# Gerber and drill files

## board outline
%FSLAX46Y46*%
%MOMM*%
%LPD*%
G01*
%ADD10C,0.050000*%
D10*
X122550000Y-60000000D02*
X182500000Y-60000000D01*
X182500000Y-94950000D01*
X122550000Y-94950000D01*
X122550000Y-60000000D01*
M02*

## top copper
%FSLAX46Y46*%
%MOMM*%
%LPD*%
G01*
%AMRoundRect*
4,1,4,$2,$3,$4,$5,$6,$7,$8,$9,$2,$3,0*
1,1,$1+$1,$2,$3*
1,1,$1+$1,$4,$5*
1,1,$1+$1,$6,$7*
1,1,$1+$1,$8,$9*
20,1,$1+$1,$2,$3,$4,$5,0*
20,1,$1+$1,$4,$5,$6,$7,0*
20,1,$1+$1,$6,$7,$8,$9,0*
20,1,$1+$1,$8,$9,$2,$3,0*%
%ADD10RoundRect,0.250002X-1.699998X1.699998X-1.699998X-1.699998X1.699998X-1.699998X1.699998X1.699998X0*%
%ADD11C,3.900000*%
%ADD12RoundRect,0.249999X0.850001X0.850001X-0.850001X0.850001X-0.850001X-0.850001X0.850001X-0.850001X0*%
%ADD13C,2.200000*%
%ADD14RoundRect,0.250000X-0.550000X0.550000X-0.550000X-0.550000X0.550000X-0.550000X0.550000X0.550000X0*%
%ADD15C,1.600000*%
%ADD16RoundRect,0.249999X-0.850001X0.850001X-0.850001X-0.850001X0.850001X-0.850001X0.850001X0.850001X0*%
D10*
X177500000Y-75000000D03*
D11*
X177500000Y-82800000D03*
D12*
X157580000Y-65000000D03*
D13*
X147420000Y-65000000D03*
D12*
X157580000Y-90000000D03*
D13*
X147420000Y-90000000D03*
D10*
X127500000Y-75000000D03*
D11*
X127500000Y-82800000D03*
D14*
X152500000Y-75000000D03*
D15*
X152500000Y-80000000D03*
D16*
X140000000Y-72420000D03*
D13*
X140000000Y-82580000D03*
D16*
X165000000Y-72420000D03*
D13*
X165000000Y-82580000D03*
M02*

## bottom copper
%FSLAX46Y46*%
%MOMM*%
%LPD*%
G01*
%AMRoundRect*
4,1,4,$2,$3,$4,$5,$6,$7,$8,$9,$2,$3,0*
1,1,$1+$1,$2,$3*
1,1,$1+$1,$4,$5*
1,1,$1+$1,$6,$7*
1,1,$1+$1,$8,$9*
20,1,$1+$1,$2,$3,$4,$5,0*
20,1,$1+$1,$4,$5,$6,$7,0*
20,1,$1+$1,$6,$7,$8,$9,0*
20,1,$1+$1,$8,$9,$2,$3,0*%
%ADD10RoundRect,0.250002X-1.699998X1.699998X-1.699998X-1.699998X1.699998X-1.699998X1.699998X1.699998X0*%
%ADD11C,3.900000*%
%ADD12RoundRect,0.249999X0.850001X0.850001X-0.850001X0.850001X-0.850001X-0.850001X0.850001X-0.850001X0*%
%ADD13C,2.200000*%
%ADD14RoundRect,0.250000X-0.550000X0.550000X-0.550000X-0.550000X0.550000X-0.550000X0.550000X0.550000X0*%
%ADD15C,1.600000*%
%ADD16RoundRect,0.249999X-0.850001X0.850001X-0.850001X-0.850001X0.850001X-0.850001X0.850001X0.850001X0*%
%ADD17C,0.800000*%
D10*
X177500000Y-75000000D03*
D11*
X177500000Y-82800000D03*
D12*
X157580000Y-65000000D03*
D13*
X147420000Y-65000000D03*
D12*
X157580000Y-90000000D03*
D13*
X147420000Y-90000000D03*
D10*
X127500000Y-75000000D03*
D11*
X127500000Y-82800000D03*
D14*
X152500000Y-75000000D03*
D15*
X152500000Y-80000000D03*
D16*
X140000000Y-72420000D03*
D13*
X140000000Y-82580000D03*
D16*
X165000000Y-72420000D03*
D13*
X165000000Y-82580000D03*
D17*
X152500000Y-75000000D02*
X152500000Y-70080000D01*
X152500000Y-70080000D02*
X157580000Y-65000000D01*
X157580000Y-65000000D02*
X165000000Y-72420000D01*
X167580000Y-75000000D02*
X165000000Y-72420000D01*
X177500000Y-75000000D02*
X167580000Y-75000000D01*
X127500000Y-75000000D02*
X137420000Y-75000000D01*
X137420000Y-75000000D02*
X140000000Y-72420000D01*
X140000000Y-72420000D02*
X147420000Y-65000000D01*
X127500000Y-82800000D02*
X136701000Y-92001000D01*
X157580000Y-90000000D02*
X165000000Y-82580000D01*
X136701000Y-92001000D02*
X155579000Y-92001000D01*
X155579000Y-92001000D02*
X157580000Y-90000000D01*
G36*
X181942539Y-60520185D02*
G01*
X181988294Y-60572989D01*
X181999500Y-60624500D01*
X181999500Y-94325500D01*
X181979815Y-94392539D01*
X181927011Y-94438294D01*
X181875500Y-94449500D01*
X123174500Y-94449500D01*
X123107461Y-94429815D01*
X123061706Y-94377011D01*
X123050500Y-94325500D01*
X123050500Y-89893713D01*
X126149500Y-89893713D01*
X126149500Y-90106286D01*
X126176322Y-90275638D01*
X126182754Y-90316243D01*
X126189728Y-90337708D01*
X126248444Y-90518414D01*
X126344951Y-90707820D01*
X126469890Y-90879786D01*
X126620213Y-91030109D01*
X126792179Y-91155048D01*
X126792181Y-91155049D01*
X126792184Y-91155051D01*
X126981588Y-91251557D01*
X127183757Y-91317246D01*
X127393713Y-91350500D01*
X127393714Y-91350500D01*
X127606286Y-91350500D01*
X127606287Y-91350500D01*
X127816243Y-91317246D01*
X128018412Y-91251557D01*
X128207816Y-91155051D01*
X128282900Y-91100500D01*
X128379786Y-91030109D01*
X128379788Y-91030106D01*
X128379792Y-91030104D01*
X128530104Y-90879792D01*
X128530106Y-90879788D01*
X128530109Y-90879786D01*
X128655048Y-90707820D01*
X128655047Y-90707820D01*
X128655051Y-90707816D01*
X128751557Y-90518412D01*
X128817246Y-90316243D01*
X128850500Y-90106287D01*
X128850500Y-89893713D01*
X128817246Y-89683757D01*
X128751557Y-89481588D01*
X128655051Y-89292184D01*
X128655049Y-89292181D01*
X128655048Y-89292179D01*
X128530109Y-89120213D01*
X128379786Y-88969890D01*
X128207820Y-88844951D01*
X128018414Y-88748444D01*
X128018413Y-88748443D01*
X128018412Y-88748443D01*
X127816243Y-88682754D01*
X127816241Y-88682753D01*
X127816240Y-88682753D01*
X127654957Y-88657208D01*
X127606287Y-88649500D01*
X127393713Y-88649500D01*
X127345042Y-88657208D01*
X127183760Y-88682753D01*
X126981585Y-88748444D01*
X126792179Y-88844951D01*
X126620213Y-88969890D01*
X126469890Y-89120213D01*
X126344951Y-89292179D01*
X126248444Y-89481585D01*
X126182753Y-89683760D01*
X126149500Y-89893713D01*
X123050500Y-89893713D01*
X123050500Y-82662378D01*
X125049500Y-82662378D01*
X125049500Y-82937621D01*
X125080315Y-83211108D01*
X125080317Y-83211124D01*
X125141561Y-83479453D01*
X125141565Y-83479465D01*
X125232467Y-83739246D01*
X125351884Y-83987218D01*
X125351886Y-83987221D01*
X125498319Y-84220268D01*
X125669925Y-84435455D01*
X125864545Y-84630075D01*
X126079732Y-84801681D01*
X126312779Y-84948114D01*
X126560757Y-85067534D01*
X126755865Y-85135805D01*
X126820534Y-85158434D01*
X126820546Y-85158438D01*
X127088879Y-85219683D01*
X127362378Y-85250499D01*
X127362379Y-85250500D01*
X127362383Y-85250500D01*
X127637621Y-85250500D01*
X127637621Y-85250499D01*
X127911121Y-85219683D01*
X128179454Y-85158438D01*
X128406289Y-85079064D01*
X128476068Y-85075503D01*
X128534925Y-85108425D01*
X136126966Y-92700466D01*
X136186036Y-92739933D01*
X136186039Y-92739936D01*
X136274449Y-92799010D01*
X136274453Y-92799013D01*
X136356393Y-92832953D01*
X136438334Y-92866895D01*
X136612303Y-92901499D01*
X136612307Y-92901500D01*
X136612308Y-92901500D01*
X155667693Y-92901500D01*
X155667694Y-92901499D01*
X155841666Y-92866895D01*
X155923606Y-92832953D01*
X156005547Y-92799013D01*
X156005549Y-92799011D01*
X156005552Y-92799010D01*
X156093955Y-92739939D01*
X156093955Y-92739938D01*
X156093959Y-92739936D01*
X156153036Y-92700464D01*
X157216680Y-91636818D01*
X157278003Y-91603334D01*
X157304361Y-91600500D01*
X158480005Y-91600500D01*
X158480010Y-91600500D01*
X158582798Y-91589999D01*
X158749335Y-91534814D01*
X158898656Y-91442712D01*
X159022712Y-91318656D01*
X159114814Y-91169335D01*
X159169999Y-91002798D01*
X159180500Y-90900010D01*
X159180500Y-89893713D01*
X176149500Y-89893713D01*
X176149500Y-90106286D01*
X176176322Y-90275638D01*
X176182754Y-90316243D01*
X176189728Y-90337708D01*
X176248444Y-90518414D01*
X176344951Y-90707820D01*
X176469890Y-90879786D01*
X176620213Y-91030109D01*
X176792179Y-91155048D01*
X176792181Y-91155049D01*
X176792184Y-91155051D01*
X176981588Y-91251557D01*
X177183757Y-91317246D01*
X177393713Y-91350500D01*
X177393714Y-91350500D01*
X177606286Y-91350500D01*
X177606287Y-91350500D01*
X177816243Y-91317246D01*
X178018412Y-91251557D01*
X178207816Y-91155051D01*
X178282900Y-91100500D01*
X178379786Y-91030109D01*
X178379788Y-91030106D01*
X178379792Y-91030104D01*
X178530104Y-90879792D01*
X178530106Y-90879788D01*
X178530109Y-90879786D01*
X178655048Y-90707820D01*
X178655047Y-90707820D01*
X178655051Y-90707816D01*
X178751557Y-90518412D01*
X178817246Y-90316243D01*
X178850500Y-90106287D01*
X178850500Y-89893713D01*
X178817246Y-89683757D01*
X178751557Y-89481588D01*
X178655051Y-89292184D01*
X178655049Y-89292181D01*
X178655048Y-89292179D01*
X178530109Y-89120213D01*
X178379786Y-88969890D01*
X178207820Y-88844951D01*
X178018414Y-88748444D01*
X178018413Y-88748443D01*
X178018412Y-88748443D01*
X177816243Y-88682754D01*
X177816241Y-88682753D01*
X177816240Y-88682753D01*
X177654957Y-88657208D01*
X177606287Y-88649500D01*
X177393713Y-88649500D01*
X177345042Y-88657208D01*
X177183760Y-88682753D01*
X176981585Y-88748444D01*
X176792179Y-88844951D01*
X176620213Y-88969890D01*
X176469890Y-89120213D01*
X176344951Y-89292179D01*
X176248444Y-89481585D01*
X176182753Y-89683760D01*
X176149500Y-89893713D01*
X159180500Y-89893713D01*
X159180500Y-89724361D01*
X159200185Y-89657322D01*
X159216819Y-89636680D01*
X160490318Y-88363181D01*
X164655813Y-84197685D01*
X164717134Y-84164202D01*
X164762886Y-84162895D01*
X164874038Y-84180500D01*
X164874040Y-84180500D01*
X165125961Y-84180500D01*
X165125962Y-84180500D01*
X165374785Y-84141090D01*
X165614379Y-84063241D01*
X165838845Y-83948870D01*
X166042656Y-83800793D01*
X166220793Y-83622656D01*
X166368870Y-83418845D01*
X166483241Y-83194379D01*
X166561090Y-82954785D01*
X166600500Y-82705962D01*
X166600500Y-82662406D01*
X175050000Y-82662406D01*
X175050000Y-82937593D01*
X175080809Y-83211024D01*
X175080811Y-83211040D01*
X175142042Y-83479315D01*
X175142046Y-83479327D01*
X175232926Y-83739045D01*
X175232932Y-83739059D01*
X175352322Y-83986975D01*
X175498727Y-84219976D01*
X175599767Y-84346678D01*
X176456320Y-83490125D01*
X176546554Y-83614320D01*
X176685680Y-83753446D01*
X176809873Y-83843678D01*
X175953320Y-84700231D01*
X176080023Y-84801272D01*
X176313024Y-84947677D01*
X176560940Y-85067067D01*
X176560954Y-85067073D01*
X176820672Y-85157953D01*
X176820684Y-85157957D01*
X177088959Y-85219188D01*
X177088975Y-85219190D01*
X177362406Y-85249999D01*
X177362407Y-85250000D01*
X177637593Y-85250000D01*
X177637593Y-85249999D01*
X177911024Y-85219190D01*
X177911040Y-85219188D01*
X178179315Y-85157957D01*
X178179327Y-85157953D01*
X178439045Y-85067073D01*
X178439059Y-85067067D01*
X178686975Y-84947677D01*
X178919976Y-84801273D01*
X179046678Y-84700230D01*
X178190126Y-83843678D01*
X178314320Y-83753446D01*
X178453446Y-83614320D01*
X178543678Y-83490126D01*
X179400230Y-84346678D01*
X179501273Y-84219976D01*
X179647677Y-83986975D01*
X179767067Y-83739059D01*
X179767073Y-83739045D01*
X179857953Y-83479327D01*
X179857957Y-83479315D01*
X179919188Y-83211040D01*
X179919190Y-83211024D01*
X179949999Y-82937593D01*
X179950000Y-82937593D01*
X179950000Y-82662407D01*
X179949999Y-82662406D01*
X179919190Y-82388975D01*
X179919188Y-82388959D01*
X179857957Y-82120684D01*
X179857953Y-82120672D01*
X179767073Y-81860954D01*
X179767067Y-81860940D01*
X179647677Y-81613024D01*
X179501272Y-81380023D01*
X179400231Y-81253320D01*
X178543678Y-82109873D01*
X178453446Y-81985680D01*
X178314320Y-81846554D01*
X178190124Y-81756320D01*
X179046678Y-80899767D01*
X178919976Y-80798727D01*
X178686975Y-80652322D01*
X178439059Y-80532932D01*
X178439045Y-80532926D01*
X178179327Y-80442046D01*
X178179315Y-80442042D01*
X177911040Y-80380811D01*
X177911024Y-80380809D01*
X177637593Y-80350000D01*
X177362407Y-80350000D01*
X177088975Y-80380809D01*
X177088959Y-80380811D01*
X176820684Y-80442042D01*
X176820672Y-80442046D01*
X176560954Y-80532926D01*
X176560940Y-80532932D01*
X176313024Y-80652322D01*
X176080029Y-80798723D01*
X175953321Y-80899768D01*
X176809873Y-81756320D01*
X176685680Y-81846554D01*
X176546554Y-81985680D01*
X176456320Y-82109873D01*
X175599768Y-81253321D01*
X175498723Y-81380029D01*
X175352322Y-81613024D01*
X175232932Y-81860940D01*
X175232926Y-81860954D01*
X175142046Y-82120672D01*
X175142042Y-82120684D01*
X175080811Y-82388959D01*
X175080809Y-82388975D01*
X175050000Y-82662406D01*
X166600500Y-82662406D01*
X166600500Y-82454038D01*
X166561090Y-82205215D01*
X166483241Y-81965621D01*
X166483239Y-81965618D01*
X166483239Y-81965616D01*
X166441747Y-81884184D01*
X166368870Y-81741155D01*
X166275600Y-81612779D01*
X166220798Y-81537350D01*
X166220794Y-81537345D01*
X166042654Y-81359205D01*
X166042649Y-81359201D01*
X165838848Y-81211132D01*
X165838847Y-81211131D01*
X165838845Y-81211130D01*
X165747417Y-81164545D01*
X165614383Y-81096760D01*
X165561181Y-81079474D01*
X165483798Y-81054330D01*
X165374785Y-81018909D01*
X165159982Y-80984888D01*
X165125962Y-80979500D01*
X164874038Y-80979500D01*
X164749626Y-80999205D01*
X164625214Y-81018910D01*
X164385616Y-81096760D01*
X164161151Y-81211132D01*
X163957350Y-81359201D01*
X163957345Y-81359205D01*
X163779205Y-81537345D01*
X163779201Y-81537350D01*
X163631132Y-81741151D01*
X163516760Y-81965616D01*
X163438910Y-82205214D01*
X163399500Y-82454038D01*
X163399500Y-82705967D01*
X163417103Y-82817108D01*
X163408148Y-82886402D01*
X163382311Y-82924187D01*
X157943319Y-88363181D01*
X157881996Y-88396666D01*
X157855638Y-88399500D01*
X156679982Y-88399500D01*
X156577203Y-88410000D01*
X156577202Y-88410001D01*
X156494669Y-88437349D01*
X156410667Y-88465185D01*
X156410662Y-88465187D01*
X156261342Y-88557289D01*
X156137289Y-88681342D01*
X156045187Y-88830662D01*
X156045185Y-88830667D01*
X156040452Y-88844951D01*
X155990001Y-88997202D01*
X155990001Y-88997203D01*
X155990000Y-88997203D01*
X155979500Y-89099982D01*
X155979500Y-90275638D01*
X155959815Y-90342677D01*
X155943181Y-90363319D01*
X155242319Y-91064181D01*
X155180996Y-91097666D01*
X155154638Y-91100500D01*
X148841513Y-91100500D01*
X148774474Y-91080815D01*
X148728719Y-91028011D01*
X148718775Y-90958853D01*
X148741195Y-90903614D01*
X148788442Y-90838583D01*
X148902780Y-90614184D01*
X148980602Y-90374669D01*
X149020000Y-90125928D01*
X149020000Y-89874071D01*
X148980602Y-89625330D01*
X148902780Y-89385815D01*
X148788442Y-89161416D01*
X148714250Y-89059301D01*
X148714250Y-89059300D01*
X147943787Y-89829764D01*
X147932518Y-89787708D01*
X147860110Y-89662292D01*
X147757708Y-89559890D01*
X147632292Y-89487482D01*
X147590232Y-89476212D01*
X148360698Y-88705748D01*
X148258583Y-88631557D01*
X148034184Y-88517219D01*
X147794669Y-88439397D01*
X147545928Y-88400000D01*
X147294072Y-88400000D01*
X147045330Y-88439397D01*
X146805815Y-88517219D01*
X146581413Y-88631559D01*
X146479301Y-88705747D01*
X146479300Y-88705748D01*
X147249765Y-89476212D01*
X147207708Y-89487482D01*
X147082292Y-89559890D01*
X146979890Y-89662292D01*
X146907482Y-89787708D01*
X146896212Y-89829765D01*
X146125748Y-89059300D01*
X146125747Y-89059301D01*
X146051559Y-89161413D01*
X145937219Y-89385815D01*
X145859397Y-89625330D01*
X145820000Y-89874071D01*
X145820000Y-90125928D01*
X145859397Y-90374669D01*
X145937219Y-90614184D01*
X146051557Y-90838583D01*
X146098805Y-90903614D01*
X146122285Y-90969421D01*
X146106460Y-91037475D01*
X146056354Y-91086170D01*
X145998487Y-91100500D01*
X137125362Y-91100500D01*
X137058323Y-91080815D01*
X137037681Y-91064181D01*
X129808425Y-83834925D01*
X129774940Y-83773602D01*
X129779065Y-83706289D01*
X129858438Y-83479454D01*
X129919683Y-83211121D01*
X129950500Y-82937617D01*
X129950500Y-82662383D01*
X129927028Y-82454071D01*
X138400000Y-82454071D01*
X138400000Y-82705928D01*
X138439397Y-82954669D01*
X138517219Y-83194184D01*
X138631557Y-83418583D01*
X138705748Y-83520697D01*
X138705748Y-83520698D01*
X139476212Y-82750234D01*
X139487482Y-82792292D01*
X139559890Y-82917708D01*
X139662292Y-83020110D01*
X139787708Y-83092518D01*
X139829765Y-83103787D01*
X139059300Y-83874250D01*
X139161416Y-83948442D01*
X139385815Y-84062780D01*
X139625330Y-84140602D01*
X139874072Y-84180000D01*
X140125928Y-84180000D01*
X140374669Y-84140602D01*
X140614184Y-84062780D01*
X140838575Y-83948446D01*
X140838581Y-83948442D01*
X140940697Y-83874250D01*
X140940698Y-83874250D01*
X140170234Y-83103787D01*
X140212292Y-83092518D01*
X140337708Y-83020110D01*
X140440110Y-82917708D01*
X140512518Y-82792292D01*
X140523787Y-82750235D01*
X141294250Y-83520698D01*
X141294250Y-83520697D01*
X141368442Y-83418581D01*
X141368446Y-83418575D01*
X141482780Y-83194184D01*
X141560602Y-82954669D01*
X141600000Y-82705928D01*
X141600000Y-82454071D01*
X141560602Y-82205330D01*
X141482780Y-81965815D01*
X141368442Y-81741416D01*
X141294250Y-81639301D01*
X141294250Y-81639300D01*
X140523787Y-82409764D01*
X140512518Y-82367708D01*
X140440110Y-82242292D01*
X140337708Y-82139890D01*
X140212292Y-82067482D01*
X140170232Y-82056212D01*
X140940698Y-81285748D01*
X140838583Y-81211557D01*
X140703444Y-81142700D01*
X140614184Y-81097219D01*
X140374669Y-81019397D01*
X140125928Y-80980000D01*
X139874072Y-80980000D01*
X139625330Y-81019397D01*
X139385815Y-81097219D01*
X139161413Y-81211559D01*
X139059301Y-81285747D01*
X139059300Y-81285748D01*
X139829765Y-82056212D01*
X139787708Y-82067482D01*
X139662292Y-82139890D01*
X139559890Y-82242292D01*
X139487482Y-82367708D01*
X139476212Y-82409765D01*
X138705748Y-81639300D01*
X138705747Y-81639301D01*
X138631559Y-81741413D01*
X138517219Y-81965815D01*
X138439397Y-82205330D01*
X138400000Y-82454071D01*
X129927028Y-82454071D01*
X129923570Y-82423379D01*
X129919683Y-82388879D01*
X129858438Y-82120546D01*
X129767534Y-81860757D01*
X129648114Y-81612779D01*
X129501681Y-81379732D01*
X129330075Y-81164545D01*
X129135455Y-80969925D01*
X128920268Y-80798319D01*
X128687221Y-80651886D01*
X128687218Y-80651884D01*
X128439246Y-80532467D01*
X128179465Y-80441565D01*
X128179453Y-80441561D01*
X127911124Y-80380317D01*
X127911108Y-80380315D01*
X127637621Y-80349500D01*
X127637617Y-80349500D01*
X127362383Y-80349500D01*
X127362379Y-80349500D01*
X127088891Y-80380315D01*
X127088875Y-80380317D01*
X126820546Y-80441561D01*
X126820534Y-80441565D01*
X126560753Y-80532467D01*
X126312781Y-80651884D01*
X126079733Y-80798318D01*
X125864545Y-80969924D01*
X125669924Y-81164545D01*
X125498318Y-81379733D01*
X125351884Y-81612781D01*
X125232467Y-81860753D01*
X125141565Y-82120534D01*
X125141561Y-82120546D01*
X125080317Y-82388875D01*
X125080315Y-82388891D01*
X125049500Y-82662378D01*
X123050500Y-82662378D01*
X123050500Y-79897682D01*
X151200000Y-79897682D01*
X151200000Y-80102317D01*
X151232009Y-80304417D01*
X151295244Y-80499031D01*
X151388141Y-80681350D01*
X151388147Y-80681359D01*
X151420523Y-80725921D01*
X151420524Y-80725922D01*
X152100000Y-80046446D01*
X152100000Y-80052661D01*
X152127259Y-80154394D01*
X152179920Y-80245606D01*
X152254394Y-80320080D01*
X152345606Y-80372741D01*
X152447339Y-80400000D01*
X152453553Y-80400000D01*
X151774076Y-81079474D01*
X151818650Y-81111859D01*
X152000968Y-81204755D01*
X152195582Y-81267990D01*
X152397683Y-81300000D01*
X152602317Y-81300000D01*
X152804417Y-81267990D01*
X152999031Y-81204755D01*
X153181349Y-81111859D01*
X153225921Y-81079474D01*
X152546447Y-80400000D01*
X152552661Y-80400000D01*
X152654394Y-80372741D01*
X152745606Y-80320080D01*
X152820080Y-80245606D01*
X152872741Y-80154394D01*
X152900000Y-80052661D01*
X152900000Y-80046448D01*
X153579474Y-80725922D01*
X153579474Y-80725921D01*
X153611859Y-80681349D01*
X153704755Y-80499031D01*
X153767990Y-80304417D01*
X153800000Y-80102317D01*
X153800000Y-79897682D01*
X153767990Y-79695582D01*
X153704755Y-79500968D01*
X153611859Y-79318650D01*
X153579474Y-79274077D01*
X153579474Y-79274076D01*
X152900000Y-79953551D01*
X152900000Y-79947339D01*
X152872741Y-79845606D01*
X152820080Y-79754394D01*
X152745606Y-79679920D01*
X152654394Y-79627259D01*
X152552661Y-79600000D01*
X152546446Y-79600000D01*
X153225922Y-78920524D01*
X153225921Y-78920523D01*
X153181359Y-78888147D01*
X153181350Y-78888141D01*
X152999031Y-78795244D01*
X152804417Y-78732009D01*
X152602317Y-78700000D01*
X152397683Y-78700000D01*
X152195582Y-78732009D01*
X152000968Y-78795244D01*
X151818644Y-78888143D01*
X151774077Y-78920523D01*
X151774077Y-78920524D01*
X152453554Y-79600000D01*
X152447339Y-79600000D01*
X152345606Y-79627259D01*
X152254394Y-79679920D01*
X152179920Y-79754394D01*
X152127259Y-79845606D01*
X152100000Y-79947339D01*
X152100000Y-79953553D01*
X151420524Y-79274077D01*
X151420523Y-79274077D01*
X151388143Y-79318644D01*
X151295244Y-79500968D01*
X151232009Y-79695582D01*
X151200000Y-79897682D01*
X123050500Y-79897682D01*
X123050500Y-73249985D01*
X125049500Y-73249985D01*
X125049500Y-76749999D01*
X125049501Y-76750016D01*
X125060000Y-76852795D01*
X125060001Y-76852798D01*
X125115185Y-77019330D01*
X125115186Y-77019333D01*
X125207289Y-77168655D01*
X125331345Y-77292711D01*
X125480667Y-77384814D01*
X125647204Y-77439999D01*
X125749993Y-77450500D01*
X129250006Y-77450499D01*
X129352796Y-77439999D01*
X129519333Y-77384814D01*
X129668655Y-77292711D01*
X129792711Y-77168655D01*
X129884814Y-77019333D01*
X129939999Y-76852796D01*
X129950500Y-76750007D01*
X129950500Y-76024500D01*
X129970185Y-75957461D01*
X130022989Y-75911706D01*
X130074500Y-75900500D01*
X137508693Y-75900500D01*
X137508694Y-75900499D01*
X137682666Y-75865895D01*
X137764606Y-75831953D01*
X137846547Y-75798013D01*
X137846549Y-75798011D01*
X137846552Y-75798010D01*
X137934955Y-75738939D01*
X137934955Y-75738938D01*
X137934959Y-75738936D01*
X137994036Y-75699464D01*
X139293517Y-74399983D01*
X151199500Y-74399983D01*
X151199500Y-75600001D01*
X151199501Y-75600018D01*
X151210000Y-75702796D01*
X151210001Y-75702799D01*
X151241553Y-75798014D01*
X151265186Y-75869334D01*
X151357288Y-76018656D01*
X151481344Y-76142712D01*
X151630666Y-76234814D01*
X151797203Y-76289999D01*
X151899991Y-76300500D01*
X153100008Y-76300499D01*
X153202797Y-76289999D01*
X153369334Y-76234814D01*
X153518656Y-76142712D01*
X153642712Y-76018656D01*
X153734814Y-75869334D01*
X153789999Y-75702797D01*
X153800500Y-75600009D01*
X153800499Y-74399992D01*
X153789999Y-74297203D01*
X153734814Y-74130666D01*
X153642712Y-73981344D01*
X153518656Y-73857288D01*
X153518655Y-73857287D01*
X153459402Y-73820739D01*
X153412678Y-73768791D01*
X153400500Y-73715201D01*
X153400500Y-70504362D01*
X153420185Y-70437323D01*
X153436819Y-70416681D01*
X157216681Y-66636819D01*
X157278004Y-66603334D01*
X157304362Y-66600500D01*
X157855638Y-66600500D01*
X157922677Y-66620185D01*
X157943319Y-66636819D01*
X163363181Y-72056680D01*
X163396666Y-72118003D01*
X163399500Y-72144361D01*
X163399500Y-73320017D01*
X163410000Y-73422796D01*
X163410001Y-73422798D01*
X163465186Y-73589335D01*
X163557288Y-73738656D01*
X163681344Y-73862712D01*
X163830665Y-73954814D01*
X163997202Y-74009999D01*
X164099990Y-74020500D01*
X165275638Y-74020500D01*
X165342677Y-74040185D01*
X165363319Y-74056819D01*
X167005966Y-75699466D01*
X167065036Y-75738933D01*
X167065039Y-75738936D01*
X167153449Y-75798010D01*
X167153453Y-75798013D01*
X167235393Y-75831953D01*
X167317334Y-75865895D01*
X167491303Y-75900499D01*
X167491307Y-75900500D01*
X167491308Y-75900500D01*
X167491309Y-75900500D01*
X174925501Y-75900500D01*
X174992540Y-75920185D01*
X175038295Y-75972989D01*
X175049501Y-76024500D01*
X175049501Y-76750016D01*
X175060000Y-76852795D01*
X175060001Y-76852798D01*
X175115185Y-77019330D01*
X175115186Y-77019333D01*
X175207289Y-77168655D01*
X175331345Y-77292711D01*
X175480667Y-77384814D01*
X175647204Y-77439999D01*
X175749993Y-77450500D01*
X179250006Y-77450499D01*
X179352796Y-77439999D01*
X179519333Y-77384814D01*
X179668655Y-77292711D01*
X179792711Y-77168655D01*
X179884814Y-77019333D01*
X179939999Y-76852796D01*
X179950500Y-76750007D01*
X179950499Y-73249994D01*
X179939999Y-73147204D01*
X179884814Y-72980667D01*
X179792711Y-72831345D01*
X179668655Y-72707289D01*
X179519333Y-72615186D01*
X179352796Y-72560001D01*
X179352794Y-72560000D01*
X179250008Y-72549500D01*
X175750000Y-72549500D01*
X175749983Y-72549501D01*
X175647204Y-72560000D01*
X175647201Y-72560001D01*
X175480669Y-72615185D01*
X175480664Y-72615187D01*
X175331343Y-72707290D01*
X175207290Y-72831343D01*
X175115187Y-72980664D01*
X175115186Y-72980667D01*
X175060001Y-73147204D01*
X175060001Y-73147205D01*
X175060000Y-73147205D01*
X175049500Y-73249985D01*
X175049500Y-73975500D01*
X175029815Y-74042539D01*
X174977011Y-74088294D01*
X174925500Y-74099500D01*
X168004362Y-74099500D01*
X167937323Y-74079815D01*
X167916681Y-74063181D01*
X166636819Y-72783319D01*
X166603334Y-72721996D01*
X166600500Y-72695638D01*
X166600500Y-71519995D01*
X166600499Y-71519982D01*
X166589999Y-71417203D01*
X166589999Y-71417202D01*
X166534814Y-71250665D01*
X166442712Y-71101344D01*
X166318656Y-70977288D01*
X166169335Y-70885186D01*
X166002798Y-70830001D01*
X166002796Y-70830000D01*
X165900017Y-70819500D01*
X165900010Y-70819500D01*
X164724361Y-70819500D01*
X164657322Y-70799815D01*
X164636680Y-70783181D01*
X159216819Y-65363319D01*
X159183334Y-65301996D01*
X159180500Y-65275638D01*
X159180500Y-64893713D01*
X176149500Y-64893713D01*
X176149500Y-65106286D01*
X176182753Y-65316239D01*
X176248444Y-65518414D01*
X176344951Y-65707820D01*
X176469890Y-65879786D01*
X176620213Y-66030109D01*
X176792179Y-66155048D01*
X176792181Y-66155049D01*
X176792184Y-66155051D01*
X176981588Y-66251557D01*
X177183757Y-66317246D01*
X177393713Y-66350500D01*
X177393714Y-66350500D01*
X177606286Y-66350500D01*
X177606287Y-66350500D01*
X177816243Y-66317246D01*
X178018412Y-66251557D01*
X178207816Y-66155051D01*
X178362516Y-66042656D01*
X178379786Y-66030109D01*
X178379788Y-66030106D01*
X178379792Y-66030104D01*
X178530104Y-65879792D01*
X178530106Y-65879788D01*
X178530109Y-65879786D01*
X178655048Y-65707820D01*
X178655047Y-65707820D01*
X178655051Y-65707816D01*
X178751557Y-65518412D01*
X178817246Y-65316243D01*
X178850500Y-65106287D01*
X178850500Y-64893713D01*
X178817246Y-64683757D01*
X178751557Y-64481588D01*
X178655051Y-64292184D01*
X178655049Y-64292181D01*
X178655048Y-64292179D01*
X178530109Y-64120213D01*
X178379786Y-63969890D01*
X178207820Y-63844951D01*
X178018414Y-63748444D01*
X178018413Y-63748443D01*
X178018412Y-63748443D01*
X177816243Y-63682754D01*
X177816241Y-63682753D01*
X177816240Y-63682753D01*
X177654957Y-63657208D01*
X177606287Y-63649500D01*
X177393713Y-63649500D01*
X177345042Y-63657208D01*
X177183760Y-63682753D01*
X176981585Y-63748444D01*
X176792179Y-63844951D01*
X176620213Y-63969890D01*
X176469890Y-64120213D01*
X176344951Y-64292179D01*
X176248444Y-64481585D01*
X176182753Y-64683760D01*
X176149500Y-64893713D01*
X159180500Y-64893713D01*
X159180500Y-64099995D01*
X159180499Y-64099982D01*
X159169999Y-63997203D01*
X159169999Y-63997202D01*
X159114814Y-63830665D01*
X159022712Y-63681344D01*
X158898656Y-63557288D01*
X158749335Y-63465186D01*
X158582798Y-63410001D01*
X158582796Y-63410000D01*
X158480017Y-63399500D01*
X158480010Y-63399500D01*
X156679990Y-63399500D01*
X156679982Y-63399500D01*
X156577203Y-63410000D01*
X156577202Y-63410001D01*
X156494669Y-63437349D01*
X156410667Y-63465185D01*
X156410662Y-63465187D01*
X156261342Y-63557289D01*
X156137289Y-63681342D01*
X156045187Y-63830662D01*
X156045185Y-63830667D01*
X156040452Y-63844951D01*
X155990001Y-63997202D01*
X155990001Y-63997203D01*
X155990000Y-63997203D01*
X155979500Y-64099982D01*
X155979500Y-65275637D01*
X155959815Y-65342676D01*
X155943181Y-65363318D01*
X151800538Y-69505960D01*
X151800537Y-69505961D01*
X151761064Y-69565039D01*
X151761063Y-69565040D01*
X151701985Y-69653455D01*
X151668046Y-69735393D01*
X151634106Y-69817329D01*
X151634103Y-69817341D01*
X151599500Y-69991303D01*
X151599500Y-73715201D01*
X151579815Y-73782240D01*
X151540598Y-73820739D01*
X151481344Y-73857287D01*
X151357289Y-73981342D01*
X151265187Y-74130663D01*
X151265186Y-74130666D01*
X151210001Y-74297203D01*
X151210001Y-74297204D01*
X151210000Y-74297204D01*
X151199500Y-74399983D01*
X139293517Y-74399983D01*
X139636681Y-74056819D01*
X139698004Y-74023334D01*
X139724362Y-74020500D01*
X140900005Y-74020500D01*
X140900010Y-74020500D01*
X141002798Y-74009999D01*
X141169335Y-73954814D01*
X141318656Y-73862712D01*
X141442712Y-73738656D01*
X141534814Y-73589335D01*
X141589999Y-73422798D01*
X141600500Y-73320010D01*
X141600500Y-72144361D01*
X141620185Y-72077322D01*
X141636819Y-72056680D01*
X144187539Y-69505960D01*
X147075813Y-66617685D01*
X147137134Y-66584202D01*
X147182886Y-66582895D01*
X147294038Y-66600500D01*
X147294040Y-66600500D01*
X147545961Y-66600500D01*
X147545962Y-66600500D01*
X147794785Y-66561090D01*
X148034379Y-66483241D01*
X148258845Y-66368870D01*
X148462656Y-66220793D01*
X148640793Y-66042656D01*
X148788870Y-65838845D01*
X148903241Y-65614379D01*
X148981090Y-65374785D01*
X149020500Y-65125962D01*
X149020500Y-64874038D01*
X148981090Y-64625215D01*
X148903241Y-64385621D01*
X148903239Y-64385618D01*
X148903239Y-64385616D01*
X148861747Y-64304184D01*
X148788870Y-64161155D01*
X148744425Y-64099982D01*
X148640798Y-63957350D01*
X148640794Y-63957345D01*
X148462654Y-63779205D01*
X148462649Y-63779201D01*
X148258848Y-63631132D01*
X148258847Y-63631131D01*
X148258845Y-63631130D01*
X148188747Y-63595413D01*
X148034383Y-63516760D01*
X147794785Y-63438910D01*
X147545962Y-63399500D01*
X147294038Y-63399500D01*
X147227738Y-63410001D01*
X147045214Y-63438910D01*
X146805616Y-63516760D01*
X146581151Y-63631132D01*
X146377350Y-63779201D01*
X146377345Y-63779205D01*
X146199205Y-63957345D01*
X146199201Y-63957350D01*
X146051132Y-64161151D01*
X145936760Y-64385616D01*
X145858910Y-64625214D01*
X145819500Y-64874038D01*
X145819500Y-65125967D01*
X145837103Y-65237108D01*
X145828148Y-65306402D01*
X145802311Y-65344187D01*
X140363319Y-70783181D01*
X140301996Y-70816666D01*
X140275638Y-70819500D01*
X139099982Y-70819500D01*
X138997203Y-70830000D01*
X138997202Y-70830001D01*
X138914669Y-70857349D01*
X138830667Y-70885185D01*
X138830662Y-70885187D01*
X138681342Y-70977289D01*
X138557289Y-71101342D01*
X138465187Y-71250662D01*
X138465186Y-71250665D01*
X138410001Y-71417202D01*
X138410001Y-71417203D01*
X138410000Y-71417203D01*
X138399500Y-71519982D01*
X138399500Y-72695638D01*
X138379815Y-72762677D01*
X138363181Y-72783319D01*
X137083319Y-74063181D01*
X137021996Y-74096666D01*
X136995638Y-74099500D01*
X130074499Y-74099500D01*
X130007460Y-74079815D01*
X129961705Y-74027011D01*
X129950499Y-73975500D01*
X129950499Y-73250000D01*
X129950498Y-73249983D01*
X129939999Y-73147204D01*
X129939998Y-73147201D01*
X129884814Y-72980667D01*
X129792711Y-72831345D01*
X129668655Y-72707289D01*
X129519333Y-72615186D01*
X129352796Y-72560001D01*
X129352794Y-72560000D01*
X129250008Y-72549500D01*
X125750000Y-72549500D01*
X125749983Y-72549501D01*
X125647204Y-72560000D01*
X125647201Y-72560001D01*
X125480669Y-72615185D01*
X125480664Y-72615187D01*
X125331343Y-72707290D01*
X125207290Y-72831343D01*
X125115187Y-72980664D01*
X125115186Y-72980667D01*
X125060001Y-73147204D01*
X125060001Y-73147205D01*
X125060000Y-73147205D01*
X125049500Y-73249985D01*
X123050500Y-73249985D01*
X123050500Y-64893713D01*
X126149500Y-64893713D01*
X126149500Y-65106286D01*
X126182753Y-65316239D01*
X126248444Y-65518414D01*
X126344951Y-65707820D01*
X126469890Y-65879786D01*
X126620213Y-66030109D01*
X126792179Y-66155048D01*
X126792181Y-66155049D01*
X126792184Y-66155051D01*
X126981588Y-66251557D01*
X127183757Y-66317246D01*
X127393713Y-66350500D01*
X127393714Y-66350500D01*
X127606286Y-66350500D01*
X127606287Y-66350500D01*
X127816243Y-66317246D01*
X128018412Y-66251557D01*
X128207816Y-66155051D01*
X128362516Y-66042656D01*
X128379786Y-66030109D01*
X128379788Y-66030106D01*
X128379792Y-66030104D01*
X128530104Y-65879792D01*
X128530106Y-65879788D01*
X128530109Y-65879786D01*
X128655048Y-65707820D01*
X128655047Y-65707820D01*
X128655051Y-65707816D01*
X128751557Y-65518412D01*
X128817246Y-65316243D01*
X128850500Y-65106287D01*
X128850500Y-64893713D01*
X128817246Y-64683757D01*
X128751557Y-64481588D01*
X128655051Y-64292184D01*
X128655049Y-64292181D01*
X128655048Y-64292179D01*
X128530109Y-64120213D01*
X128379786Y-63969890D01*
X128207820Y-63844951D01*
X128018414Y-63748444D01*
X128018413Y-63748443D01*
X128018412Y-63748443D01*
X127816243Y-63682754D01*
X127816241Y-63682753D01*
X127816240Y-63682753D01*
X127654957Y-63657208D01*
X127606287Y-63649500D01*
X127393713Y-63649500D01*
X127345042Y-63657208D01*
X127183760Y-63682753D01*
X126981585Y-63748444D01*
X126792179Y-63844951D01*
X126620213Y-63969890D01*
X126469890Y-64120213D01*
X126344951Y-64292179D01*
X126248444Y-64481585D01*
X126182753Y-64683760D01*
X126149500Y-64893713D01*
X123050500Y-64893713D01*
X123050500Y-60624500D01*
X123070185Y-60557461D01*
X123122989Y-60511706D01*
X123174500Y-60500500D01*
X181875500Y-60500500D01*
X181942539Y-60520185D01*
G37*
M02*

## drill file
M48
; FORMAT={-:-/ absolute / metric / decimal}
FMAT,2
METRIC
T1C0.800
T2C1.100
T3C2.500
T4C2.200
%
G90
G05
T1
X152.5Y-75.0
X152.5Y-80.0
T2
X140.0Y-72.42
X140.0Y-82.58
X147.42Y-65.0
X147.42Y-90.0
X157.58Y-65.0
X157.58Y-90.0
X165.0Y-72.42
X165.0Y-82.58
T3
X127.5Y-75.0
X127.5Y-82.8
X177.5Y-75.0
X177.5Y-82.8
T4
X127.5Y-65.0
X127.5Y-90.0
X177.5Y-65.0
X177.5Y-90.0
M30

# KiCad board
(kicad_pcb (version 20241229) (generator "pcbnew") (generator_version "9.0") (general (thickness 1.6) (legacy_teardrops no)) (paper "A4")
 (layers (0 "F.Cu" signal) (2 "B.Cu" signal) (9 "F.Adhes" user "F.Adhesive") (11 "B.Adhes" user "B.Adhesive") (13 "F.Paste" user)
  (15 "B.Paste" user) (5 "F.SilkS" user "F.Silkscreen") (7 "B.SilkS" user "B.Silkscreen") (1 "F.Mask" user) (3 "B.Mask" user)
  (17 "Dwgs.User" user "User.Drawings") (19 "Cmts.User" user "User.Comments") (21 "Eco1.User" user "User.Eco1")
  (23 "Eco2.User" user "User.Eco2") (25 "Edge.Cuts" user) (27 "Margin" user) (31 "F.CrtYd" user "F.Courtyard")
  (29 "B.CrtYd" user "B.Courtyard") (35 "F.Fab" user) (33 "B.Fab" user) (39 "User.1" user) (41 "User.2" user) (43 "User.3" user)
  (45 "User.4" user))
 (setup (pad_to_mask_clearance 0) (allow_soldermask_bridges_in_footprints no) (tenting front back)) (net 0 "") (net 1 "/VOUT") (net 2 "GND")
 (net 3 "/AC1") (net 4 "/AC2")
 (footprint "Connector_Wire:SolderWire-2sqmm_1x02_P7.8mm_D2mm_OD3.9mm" (layer "F.Cu") (at 177.5 75 -90)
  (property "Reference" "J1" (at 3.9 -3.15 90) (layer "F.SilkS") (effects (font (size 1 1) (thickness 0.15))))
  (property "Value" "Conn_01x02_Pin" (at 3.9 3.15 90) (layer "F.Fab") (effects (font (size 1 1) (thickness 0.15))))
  (pad "1" thru_hole roundrect (at 0 0 270) (size 3.9 3.9) (drill 2.5) (layers "*.Cu" "*.Mask") (remove_unused_layers no)
   (roundrect_rratio 0.064103) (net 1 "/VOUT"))
  (pad "2" thru_hole circle (at 7.8 0 270) (size 3.9 3.9) (drill 2.5) (layers "*.Cu" "*.Mask") (remove_unused_layers no) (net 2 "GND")))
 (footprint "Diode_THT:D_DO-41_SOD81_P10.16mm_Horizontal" (layer "F.Cu") (at 157.58 65 180)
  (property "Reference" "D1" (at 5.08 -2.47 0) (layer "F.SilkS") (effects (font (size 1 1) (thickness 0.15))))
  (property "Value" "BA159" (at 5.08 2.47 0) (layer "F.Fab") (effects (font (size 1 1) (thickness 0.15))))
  (pad "1" thru_hole roundrect (at 0 0 180) (size 2.2 2.2) (drill 1.1) (layers "*.Cu" "*.Mask") (remove_unused_layers no)
   (roundrect_rratio 0.113636) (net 1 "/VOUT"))
  (pad "2" thru_hole circle (at 10.16 0 180) (size 2.2 2.2) (drill 1.1) (layers "*.Cu" "*.Mask") (remove_unused_layers no) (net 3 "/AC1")))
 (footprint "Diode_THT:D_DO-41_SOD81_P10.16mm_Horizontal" (layer "F.Cu") (at 157.58 90 180)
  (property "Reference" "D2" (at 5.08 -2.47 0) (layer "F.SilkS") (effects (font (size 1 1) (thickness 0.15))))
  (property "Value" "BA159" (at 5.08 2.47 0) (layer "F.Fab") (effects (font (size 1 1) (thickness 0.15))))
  (pad "1" thru_hole roundrect (at 0 0 180) (size 2.2 2.2) (drill 1.1) (layers "*.Cu" "*.Mask") (remove_unused_layers no)
   (roundrect_rratio 0.113636) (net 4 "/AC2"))
  (pad "2" thru_hole circle (at 10.16 0 180) (size 2.2 2.2) (drill 1.1) (layers "*.Cu" "*.Mask") (remove_unused_layers no) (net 2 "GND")))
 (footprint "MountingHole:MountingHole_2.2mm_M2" (layer "F.Cu") (at 127.5 65)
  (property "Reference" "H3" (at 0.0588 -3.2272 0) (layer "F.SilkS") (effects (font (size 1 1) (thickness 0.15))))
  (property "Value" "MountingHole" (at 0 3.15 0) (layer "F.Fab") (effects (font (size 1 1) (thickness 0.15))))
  (pad "" np_thru_hole circle (at 0 0) (size 2.2 2.2) (drill 2.2) (layers "*.Cu" "*.Mask")))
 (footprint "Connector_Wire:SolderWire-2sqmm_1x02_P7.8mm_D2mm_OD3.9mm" (layer "F.Cu") (at 127.5 75 -90)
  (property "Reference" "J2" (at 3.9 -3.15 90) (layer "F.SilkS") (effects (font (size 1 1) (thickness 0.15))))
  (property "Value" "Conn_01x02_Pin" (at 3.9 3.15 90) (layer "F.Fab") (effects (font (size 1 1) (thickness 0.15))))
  (pad "1" thru_hole roundrect (at 0 0 270) (size 3.9 3.9) (drill 2.5) (layers "*.Cu" "*.Mask") (remove_unused_layers no)
   (roundrect_rratio 0.064103) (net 3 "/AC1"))
  (pad "2" thru_hole circle (at 7.8 0 270) (size 3.9 3.9) (drill 2.5) (layers "*.Cu" "*.Mask") (remove_unused_layers no) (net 4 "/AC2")))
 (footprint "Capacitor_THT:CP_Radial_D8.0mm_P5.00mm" (layer "F.Cu") (at 152.5 75 -90)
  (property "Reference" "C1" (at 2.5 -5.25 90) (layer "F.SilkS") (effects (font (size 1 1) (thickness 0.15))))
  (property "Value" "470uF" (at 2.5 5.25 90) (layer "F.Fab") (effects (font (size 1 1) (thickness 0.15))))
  (pad "1" thru_hole roundrect (at 0 0 270) (size 1.6 1.6) (drill 0.8) (layers "*.Cu" "*.Mask") (remove_unused_layers no)
   (roundrect_rratio 0.15625) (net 1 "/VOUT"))
  (pad "2" thru_hole circle (at 5 0 270) (size 1.6 1.6) (drill 0.8) (layers "*.Cu" "*.Mask") (remove_unused_layers no) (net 2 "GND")))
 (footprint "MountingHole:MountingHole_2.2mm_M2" (layer "F.Cu") (at 177.5 90)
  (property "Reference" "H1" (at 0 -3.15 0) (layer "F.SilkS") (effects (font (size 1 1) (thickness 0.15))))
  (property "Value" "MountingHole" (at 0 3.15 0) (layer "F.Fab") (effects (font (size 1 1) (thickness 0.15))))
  (pad "" np_thru_hole circle (at 0 0) (size 2.2 2.2) (drill 2.2) (layers "*.Cu" "*.Mask")))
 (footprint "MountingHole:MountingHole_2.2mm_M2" (layer "F.Cu") (at 127.5 90)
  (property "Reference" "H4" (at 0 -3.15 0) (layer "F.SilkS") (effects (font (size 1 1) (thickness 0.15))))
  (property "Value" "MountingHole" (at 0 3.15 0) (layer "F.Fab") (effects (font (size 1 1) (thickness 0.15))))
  (pad "" np_thru_hole circle (at 0 0) (size 2.2 2.2) (drill 2.2) (layers "*.Cu" "*.Mask")))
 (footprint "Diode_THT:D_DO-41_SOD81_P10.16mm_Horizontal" (layer "F.Cu") (at 140 72.42 -90)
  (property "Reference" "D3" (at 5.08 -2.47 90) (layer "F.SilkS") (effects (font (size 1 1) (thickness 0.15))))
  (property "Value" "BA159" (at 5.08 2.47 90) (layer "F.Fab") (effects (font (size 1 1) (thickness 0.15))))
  (pad "1" thru_hole roundrect (at 0 0 270) (size 2.2 2.2) (drill 1.1) (layers "*.Cu" "*.Mask") (remove_unused_layers no)
   (roundrect_rratio 0.113636) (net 3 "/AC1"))
  (pad "2" thru_hole circle (at 10.16 0 270) (size 2.2 2.2) (drill 1.1) (layers "*.Cu" "*.Mask") (remove_unused_layers no) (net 2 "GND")))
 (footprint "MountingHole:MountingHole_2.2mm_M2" (layer "F.Cu") (at 177.5 65)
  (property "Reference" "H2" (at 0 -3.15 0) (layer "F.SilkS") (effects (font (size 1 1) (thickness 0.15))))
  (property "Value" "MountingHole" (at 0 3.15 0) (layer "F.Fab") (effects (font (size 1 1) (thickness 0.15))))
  (pad "" np_thru_hole circle (at 0 0) (size 2.2 2.2) (drill 2.2) (layers "*.Cu" "*.Mask")))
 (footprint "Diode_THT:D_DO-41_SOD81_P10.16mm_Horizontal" (layer "F.Cu") (at 165 72.42 -90)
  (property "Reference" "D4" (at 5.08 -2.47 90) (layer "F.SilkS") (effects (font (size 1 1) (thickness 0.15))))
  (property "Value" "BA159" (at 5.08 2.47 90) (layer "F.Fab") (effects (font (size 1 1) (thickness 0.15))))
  (pad "1" thru_hole roundrect (at 0 0 270) (size 2.2 2.2) (drill 1.1) (layers "*.Cu" "*.Mask") (remove_unused_layers no)
   (roundrect_rratio 0.113636) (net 1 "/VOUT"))
  (pad "2" thru_hole circle (at 10.16 0 270) (size 2.2 2.2) (drill 1.1) (layers "*.Cu" "*.Mask") (remove_unused_layers no) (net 4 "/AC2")))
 (gr_rect (start 122.55 60) (end 182.5 94.95) (stroke (width 0.05) (type default)) (fill no) (layer "Edge.Cuts"))
 (segment (start 152.5 75) (end 152.5 70.08) (width 0.8) (layer "B.Cu") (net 1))
 (segment (start 152.5 70.08) (end 157.58 65) (width 0.8) (layer "B.Cu") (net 1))
 (segment (start 157.58 65) (end 165 72.42) (width 0.8) (layer "B.Cu") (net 1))
 (segment (start 167.58 75) (end 165 72.42) (width 0.8) (layer "B.Cu") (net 1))
 (segment (start 177.5 75) (end 167.58 75) (width 0.8) (layer "B.Cu") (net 1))
 (segment (start 127.5 75) (end 137.42 75) (width 0.8) (layer "B.Cu") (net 3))
 (segment (start 137.42 75) (end 140 72.42) (width 0.8) (layer "B.Cu") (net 3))
 (segment (start 140 72.42) (end 147.42 65) (width 0.8) (layer "B.Cu") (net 3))
 (segment (start 127.5 82.8) (end 136.701 92.001) (width 0.8) (layer "B.Cu") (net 4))
 (segment (start 157.58 90) (end 165 82.58) (width 0.8) (layer "B.Cu") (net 4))
 (segment (start 136.701 92.001) (end 155.579 92.001) (width 0.8) (layer "B.Cu") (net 4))
 (segment (start 155.579 92.001) (end 157.58 90) (width 0.8) (layer "B.Cu") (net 4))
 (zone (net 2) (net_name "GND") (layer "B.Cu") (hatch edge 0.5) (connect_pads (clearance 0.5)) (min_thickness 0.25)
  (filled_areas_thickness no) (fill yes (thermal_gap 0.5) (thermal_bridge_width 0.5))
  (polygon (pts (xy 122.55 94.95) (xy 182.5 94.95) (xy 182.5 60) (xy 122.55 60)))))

